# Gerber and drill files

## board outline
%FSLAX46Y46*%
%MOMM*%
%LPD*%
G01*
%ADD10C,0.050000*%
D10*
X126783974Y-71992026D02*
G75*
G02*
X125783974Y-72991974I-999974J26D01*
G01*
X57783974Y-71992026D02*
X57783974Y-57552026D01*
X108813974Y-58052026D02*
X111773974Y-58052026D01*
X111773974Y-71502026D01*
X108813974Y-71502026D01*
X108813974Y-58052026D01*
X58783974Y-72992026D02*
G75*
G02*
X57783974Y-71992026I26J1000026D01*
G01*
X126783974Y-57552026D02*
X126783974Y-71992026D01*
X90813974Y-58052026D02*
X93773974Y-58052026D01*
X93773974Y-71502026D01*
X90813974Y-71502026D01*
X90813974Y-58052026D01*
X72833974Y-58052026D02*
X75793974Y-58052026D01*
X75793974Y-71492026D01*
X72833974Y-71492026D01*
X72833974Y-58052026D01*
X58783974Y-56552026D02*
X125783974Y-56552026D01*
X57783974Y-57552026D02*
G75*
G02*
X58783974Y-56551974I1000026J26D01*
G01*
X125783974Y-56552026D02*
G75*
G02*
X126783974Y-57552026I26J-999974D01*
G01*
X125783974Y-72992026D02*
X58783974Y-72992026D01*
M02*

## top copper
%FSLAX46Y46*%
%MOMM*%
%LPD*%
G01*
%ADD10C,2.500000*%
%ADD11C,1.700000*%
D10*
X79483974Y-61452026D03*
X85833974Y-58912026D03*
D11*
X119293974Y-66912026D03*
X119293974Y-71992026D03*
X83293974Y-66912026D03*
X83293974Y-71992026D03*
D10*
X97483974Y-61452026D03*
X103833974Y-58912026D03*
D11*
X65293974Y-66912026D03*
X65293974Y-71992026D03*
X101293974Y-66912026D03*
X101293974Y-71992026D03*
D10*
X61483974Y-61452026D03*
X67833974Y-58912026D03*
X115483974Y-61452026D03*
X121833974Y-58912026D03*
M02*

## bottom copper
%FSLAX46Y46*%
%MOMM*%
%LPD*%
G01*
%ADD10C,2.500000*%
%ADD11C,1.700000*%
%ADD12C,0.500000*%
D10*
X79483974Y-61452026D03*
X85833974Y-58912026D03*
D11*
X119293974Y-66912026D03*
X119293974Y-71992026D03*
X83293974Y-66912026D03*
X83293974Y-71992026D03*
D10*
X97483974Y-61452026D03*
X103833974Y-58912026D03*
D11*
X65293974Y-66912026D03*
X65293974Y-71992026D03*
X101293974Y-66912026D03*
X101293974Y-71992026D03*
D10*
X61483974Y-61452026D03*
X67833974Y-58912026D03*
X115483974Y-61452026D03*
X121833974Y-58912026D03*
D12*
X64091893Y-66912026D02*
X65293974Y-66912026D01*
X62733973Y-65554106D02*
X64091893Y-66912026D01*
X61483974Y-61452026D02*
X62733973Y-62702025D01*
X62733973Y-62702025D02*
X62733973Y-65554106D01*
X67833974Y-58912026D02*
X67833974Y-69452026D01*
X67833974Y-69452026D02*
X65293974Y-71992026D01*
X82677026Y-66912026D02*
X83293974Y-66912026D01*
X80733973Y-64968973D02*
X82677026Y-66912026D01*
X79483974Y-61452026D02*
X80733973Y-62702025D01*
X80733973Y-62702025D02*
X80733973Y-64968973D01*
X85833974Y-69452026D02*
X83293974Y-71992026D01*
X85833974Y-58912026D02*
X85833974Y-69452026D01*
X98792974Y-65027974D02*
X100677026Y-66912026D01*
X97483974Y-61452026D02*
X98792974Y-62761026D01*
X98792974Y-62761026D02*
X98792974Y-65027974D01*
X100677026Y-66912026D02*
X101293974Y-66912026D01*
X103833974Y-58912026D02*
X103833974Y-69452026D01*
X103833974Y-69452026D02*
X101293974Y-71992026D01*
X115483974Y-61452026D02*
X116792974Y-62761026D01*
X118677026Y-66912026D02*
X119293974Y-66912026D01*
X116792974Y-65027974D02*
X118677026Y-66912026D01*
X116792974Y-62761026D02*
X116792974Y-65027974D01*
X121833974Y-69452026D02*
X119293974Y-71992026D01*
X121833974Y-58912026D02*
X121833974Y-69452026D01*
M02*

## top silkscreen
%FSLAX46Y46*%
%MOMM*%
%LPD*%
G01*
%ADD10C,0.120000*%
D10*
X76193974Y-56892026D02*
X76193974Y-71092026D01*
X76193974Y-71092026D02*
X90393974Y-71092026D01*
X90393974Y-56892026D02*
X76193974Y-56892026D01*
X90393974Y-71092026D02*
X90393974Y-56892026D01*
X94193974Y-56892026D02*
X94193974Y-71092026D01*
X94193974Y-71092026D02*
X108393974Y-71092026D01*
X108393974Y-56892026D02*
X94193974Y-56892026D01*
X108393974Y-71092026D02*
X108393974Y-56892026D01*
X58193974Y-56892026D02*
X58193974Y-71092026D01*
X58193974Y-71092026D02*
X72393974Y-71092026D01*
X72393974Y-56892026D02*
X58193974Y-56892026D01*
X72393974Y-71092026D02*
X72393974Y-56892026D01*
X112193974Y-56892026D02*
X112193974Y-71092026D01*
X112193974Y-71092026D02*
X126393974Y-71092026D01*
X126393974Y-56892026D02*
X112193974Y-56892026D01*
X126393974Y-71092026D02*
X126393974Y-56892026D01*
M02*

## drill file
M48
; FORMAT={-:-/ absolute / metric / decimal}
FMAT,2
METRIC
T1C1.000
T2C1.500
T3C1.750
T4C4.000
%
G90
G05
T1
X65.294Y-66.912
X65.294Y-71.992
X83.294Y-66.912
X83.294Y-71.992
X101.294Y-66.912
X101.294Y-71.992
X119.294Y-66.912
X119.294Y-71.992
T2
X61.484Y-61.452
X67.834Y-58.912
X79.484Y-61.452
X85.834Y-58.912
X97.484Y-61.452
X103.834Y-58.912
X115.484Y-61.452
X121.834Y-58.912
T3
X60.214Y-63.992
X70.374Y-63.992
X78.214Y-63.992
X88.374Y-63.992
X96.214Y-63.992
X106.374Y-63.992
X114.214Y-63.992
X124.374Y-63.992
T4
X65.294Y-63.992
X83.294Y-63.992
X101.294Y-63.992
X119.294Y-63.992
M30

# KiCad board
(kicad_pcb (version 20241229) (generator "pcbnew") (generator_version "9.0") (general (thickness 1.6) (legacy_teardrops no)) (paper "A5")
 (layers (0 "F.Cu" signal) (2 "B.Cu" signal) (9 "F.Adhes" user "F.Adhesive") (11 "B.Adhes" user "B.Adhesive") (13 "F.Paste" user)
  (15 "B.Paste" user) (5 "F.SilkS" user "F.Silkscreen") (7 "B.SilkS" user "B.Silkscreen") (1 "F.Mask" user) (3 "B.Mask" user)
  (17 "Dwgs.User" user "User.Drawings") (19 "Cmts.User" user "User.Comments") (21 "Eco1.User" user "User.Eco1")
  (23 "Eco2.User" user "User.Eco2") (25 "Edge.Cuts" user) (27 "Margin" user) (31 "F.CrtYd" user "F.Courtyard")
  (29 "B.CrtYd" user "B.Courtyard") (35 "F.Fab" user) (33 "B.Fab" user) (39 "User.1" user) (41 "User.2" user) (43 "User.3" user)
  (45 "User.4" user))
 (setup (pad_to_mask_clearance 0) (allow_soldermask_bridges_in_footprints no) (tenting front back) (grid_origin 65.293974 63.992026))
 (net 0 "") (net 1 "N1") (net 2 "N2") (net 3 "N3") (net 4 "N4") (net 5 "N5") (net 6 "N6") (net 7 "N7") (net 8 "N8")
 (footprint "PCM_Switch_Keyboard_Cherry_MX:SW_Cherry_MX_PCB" (layer "F.Cu") (at 83.293974 63.992026)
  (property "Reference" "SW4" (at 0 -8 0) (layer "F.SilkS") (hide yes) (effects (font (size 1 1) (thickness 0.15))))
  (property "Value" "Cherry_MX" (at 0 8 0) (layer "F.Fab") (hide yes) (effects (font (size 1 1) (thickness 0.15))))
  (fp_line (start -7.1 -7.1) (end -7.1 7.1) (stroke (width 0.12) (type solid)) (layer "F.SilkS"))
  (fp_line (start -7.1 7.1) (end 7.1 7.1) (stroke (width 0.12) (type solid)) (layer "F.SilkS"))
  (fp_line (start 7.1 -7.1) (end -7.1 -7.1) (stroke (width 0.12) (type solid)) (layer "F.SilkS"))
  (fp_line (start 7.1 7.1) (end 7.1 -7.1) (stroke (width 0.12) (type solid)) (layer "F.SilkS"))
  (pad "" np_thru_hole circle (at -5.08 0) (size 1.75 1.75) (drill 1.75) (layers "*.Cu" "*.Mask"))
  (pad "" np_thru_hole circle (at 0 0) (size 4 4) (drill 4) (layers "*.Cu" "*.Mask"))
  (pad "" np_thru_hole circle (at 5.08 0) (size 1.75 1.75) (drill 1.75) (layers "*.Cu" "*.Mask"))
  (pad "1" thru_hole circle (at -3.81 -2.54) (size 2.5 2.5) (drill 1.5) (layers "*.Cu" "*.Mask") (remove_unused_layers no) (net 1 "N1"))
  (pad "2" thru_hole circle (at 2.54 -5.08) (size 2.5 2.5) (drill 1.5) (layers "*.Cu" "*.Mask") (remove_unused_layers no) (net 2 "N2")))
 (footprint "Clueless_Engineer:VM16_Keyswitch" (layer "F.Cu") (at 119.293974 71.992026)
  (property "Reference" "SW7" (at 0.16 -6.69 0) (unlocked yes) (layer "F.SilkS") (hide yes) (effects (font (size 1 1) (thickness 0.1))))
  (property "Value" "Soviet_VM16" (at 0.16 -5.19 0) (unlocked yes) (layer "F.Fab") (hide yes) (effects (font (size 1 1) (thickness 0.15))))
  (pad "1" thru_hole circle (at 0 -5.08) (size 1.7 1.7) (drill 1) (layers "*.Cu" "*.Mask") (remove_unused_layers no) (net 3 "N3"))
  (pad "2" thru_hole circle (at 0 0) (size 1.7 1.7) (drill 1) (layers "*.Cu" "*.Mask") (remove_unused_layers no) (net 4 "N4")))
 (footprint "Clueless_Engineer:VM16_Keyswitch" (layer "F.Cu") (at 83.293974 71.992026)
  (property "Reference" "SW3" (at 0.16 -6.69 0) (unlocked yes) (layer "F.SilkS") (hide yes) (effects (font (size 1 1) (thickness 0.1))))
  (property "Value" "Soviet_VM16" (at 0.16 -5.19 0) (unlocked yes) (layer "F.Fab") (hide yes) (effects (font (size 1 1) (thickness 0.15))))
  (pad "1" thru_hole circle (at 0 -5.08) (size 1.7 1.7) (drill 1) (layers "*.Cu" "*.Mask") (remove_unused_layers no) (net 1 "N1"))
  (pad "2" thru_hole circle (at 0 0) (size 1.7 1.7) (drill 1) (layers "*.Cu" "*.Mask") (remove_unused_layers no) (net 2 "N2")))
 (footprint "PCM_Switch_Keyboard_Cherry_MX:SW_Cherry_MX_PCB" (layer "F.Cu") (at 101.293974 63.992026)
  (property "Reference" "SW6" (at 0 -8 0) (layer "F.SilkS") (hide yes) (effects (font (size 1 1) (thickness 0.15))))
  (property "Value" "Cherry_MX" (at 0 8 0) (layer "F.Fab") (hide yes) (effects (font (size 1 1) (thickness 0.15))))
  (fp_line (start -7.1 -7.1) (end -7.1 7.1) (stroke (width 0.12) (type solid)) (layer "F.SilkS"))
  (fp_line (start -7.1 7.1) (end 7.1 7.1) (stroke (width 0.12) (type solid)) (layer "F.SilkS"))
  (fp_line (start 7.1 -7.1) (end -7.1 -7.1) (stroke (width 0.12) (type solid)) (layer "F.SilkS"))
  (fp_line (start 7.1 7.1) (end 7.1 -7.1) (stroke (width 0.12) (type solid)) (layer "F.SilkS"))
  (pad "" np_thru_hole circle (at -5.08 0) (size 1.75 1.75) (drill 1.75) (layers "*.Cu" "*.Mask"))
  (pad "" np_thru_hole circle (at 0 0) (size 4 4) (drill 4) (layers "*.Cu" "*.Mask"))
  (pad "" np_thru_hole circle (at 5.08 0) (size 1.75 1.75) (drill 1.75) (layers "*.Cu" "*.Mask"))
  (pad "1" thru_hole circle (at -3.81 -2.54) (size 2.5 2.5) (drill 1.5) (layers "*.Cu" "*.Mask") (remove_unused_layers no) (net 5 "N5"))
  (pad "2" thru_hole circle (at 2.54 -5.08) (size 2.5 2.5) (drill 1.5) (layers "*.Cu" "*.Mask") (remove_unused_layers no) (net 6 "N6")))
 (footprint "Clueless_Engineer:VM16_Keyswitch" (layer "F.Cu") (at 65.293974 71.992026)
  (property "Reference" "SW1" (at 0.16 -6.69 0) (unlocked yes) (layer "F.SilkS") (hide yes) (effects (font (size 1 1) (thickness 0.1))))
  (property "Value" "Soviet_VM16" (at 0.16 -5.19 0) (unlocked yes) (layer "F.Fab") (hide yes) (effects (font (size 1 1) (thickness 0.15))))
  (pad "1" thru_hole circle (at 0 -5.08) (size 1.7 1.7) (drill 1) (layers "*.Cu" "*.Mask") (remove_unused_layers no) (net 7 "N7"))
  (pad "2" thru_hole circle (at 0 0) (size 1.7 1.7) (drill 1) (layers "*.Cu" "*.Mask") (remove_unused_layers no) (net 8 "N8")))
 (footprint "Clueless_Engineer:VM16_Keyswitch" (layer "F.Cu") (at 101.293974 71.992026)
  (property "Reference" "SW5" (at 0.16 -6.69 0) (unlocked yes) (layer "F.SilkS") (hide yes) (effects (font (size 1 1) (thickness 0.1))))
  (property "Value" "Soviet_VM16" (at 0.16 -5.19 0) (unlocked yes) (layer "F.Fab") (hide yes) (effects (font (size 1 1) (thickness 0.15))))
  (pad "1" thru_hole circle (at 0 -5.08) (size 1.7 1.7) (drill 1) (layers "*.Cu" "*.Mask") (remove_unused_layers no) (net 5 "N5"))
  (pad "2" thru_hole circle (at 0 0) (size 1.7 1.7) (drill 1) (layers "*.Cu" "*.Mask") (remove_unused_layers no) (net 6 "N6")))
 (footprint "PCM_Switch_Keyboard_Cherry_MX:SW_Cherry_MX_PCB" (layer "F.Cu") (at 65.293974 63.992026)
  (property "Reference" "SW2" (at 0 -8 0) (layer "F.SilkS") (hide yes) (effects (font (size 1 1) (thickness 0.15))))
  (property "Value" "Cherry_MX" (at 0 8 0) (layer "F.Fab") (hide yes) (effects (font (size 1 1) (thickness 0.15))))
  (fp_line (start -7.1 -7.1) (end -7.1 7.1) (stroke (width 0.12) (type solid)) (layer "F.SilkS"))
  (fp_line (start -7.1 7.1) (end 7.1 7.1) (stroke (width 0.12) (type solid)) (layer "F.SilkS"))
  (fp_line (start 7.1 -7.1) (end -7.1 -7.1) (stroke (width 0.12) (type solid)) (layer "F.SilkS"))
  (fp_line (start 7.1 7.1) (end 7.1 -7.1) (stroke (width 0.12) (type solid)) (layer "F.SilkS"))
  (pad "" np_thru_hole circle (at -5.08 0) (size 1.75 1.75) (drill 1.75) (layers "*.Cu" "*.Mask"))
  (pad "" np_thru_hole circle (at 0 0) (size 4 4) (drill 4) (layers "*.Cu" "*.Mask"))
  (pad "" np_thru_hole circle (at 5.08 0) (size 1.75 1.75) (drill 1.75) (layers "*.Cu" "*.Mask"))
  (pad "1" thru_hole circle (at -3.81 -2.54) (size 2.5 2.5) (drill 1.5) (layers "*.Cu" "*.Mask") (remove_unused_layers no) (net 7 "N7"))
  (pad "2" thru_hole circle (at 2.54 -5.08) (size 2.5 2.5) (drill 1.5) (layers "*.Cu" "*.Mask") (remove_unused_layers no) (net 8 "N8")))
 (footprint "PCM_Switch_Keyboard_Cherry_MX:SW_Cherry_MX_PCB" (layer "F.Cu") (at 119.293974 63.992026)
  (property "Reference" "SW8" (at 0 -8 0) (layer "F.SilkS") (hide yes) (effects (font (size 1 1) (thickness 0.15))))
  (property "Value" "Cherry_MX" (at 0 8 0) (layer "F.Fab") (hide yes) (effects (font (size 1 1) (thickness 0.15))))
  (fp_line (start -7.1 -7.1) (end -7.1 7.1) (stroke (width 0.12) (type solid)) (layer "F.SilkS"))
  (fp_line (start -7.1 7.1) (end 7.1 7.1) (stroke (width 0.12) (type solid)) (layer "F.SilkS"))
  (fp_line (start 7.1 -7.1) (end -7.1 -7.1) (stroke (width 0.12) (type solid)) (layer "F.SilkS"))
  (fp_line (start 7.1 7.1) (end 7.1 -7.1) (stroke (width 0.12) (type solid)) (layer "F.SilkS"))
  (pad "" np_thru_hole circle (at -5.08 0) (size 1.75 1.75) (drill 1.75) (layers "*.Cu" "*.Mask"))
  (pad "" np_thru_hole circle (at 0 0) (size 4 4) (drill 4) (layers "*.Cu" "*.Mask"))
  (pad "" np_thru_hole circle (at 5.08 0) (size 1.75 1.75) (drill 1.75) (layers "*.Cu" "*.Mask"))
  (pad "1" thru_hole circle (at -3.81 -2.54) (size 2.5 2.5) (drill 1.5) (layers "*.Cu" "*.Mask") (remove_unused_layers no) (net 3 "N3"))
  (pad "2" thru_hole circle (at 2.54 -5.08) (size 2.5 2.5) (drill 1.5) (layers "*.Cu" "*.Mask") (remove_unused_layers no) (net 4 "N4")))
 (gr_arc (start 126.783974 71.992026) (mid 126.491081 72.699133) (end 125.783974 72.992026) (stroke (width 0.05) (type default))
  (layer "Edge.Cuts"))
 (gr_line (start 57.783974 71.992026) (end 57.783974 57.552026) (stroke (width 0.05) (type default)) (layer "Edge.Cuts"))
 (gr_rect (start 108.813974 58.052026) (end 111.773974 71.502026) (stroke (width 0.05) (type solid)) (fill no) (layer "Edge.Cuts"))
 (gr_arc (start 58.783974 72.992026) (mid 58.076867 72.699133) (end 57.783974 71.992026) (stroke (width 0.05) (type default))
  (layer "Edge.Cuts"))
 (gr_line (start 126.783974 57.552026) (end 126.783974 71.992026) (stroke (width 0.05) (type default)) (layer "Edge.Cuts"))
 (gr_rect (start 90.813974 58.052026) (end 93.773974 71.502026) (stroke (width 0.05) (type solid)) (fill no) (layer "Edge.Cuts"))
 (gr_rect (start 72.833974 58.052026) (end 75.793974 71.492026) (stroke (width 0.05) (type solid)) (fill no) (layer "Edge.Cuts"))
 (gr_line (start 58.783974 56.552026) (end 125.783974 56.552026) (stroke (width 0.05) (type default)) (layer "Edge.Cuts"))
 (gr_arc (start 57.783974 57.552026) (mid 58.076867 56.844919) (end 58.783974 56.552026) (stroke (width 0.05) (type default))
  (layer "Edge.Cuts"))
 (gr_arc (start 125.783974 56.552026) (mid 126.491081 56.844919) (end 126.783974 57.552026) (stroke (width 0.05) (type default))
  (layer "Edge.Cuts"))
 (gr_line (start 125.783974 72.992026) (end 58.783974 72.992026) (stroke (width 0.05) (type default)) (layer "Edge.Cuts"))
 (segment (start 64.091893 66.912026) (end 65.293974 66.912026) (width 0.5) (layer "B.Cu") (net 7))
 (segment (start 62.733973 65.554106) (end 64.091893 66.912026) (width 0.5) (layer "B.Cu") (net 7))
 (segment (start 61.483974 61.452026) (end 62.733973 62.702025) (width 0.5) (layer "B.Cu") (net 7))
 (segment (start 62.733973 62.702025) (end 62.733973 65.554106) (width 0.5) (layer "B.Cu") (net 7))
 (segment (start 67.833974 58.912026) (end 67.833974 69.452026) (width 0.5) (layer "B.Cu") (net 8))
 (segment (start 67.833974 69.452026) (end 65.293974 71.992026) (width 0.5) (layer "B.Cu") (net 8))
 (segment (start 82.677026 66.912026) (end 83.293974 66.912026) (width 0.5) (layer "B.Cu") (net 1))
 (segment (start 80.733973 64.968973) (end 82.677026 66.912026) (width 0.5) (layer "B.Cu") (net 1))
 (segment (start 79.483974 61.452026) (end 80.733973 62.702025) (width 0.5) (layer "B.Cu") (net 1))
 (segment (start 80.733973 62.702025) (end 80.733973 64.968973) (width 0.5) (layer "B.Cu") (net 1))
 (segment (start 85.833974 69.452026) (end 83.293974 71.992026) (width 0.5) (layer "B.Cu") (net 2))
 (segment (start 85.833974 58.912026) (end 85.833974 69.452026) (width 0.5) (layer "B.Cu") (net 2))
 (segment (start 98.792974 65.027974) (end 100.677026 66.912026) (width 0.5) (layer "B.Cu") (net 5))
 (segment (start 97.483974 61.452026) (end 98.792974 62.761026) (width 0.5) (layer "B.Cu") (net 5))
 (segment (start 98.792974 62.761026) (end 98.792974 65.027974) (width 0.5) (layer "B.Cu") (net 5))
 (segment (start 100.677026 66.912026) (end 101.293974 66.912026) (width 0.5) (layer "B.Cu") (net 5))
 (segment (start 103.833974 58.912026) (end 103.833974 69.452026) (width 0.5) (layer "B.Cu") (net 6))
 (segment (start 103.833974 69.452026) (end 101.293974 71.992026) (width 0.5) (layer "B.Cu") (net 6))
 (segment (start 115.483974 61.452026) (end 116.792974 62.761026) (width 0.5) (layer "B.Cu") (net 3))
 (segment (start 118.677026 66.912026) (end 119.293974 66.912026) (width 0.5) (layer "B.Cu") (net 3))
 (segment (start 116.792974 65.027974) (end 118.677026 66.912026) (width 0.5) (layer "B.Cu") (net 3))
 (segment (start 116.792974 62.761026) (end 116.792974 65.027974) (width 0.5) (layer "B.Cu") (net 3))
 (segment (start 121.833974 69.452026) (end 119.293974 71.992026) (width 0.5) (layer "B.Cu") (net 4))
 (segment (start 121.833974 58.912026) (end 121.833974 69.452026) (width 0.5) (layer "B.Cu") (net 4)))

